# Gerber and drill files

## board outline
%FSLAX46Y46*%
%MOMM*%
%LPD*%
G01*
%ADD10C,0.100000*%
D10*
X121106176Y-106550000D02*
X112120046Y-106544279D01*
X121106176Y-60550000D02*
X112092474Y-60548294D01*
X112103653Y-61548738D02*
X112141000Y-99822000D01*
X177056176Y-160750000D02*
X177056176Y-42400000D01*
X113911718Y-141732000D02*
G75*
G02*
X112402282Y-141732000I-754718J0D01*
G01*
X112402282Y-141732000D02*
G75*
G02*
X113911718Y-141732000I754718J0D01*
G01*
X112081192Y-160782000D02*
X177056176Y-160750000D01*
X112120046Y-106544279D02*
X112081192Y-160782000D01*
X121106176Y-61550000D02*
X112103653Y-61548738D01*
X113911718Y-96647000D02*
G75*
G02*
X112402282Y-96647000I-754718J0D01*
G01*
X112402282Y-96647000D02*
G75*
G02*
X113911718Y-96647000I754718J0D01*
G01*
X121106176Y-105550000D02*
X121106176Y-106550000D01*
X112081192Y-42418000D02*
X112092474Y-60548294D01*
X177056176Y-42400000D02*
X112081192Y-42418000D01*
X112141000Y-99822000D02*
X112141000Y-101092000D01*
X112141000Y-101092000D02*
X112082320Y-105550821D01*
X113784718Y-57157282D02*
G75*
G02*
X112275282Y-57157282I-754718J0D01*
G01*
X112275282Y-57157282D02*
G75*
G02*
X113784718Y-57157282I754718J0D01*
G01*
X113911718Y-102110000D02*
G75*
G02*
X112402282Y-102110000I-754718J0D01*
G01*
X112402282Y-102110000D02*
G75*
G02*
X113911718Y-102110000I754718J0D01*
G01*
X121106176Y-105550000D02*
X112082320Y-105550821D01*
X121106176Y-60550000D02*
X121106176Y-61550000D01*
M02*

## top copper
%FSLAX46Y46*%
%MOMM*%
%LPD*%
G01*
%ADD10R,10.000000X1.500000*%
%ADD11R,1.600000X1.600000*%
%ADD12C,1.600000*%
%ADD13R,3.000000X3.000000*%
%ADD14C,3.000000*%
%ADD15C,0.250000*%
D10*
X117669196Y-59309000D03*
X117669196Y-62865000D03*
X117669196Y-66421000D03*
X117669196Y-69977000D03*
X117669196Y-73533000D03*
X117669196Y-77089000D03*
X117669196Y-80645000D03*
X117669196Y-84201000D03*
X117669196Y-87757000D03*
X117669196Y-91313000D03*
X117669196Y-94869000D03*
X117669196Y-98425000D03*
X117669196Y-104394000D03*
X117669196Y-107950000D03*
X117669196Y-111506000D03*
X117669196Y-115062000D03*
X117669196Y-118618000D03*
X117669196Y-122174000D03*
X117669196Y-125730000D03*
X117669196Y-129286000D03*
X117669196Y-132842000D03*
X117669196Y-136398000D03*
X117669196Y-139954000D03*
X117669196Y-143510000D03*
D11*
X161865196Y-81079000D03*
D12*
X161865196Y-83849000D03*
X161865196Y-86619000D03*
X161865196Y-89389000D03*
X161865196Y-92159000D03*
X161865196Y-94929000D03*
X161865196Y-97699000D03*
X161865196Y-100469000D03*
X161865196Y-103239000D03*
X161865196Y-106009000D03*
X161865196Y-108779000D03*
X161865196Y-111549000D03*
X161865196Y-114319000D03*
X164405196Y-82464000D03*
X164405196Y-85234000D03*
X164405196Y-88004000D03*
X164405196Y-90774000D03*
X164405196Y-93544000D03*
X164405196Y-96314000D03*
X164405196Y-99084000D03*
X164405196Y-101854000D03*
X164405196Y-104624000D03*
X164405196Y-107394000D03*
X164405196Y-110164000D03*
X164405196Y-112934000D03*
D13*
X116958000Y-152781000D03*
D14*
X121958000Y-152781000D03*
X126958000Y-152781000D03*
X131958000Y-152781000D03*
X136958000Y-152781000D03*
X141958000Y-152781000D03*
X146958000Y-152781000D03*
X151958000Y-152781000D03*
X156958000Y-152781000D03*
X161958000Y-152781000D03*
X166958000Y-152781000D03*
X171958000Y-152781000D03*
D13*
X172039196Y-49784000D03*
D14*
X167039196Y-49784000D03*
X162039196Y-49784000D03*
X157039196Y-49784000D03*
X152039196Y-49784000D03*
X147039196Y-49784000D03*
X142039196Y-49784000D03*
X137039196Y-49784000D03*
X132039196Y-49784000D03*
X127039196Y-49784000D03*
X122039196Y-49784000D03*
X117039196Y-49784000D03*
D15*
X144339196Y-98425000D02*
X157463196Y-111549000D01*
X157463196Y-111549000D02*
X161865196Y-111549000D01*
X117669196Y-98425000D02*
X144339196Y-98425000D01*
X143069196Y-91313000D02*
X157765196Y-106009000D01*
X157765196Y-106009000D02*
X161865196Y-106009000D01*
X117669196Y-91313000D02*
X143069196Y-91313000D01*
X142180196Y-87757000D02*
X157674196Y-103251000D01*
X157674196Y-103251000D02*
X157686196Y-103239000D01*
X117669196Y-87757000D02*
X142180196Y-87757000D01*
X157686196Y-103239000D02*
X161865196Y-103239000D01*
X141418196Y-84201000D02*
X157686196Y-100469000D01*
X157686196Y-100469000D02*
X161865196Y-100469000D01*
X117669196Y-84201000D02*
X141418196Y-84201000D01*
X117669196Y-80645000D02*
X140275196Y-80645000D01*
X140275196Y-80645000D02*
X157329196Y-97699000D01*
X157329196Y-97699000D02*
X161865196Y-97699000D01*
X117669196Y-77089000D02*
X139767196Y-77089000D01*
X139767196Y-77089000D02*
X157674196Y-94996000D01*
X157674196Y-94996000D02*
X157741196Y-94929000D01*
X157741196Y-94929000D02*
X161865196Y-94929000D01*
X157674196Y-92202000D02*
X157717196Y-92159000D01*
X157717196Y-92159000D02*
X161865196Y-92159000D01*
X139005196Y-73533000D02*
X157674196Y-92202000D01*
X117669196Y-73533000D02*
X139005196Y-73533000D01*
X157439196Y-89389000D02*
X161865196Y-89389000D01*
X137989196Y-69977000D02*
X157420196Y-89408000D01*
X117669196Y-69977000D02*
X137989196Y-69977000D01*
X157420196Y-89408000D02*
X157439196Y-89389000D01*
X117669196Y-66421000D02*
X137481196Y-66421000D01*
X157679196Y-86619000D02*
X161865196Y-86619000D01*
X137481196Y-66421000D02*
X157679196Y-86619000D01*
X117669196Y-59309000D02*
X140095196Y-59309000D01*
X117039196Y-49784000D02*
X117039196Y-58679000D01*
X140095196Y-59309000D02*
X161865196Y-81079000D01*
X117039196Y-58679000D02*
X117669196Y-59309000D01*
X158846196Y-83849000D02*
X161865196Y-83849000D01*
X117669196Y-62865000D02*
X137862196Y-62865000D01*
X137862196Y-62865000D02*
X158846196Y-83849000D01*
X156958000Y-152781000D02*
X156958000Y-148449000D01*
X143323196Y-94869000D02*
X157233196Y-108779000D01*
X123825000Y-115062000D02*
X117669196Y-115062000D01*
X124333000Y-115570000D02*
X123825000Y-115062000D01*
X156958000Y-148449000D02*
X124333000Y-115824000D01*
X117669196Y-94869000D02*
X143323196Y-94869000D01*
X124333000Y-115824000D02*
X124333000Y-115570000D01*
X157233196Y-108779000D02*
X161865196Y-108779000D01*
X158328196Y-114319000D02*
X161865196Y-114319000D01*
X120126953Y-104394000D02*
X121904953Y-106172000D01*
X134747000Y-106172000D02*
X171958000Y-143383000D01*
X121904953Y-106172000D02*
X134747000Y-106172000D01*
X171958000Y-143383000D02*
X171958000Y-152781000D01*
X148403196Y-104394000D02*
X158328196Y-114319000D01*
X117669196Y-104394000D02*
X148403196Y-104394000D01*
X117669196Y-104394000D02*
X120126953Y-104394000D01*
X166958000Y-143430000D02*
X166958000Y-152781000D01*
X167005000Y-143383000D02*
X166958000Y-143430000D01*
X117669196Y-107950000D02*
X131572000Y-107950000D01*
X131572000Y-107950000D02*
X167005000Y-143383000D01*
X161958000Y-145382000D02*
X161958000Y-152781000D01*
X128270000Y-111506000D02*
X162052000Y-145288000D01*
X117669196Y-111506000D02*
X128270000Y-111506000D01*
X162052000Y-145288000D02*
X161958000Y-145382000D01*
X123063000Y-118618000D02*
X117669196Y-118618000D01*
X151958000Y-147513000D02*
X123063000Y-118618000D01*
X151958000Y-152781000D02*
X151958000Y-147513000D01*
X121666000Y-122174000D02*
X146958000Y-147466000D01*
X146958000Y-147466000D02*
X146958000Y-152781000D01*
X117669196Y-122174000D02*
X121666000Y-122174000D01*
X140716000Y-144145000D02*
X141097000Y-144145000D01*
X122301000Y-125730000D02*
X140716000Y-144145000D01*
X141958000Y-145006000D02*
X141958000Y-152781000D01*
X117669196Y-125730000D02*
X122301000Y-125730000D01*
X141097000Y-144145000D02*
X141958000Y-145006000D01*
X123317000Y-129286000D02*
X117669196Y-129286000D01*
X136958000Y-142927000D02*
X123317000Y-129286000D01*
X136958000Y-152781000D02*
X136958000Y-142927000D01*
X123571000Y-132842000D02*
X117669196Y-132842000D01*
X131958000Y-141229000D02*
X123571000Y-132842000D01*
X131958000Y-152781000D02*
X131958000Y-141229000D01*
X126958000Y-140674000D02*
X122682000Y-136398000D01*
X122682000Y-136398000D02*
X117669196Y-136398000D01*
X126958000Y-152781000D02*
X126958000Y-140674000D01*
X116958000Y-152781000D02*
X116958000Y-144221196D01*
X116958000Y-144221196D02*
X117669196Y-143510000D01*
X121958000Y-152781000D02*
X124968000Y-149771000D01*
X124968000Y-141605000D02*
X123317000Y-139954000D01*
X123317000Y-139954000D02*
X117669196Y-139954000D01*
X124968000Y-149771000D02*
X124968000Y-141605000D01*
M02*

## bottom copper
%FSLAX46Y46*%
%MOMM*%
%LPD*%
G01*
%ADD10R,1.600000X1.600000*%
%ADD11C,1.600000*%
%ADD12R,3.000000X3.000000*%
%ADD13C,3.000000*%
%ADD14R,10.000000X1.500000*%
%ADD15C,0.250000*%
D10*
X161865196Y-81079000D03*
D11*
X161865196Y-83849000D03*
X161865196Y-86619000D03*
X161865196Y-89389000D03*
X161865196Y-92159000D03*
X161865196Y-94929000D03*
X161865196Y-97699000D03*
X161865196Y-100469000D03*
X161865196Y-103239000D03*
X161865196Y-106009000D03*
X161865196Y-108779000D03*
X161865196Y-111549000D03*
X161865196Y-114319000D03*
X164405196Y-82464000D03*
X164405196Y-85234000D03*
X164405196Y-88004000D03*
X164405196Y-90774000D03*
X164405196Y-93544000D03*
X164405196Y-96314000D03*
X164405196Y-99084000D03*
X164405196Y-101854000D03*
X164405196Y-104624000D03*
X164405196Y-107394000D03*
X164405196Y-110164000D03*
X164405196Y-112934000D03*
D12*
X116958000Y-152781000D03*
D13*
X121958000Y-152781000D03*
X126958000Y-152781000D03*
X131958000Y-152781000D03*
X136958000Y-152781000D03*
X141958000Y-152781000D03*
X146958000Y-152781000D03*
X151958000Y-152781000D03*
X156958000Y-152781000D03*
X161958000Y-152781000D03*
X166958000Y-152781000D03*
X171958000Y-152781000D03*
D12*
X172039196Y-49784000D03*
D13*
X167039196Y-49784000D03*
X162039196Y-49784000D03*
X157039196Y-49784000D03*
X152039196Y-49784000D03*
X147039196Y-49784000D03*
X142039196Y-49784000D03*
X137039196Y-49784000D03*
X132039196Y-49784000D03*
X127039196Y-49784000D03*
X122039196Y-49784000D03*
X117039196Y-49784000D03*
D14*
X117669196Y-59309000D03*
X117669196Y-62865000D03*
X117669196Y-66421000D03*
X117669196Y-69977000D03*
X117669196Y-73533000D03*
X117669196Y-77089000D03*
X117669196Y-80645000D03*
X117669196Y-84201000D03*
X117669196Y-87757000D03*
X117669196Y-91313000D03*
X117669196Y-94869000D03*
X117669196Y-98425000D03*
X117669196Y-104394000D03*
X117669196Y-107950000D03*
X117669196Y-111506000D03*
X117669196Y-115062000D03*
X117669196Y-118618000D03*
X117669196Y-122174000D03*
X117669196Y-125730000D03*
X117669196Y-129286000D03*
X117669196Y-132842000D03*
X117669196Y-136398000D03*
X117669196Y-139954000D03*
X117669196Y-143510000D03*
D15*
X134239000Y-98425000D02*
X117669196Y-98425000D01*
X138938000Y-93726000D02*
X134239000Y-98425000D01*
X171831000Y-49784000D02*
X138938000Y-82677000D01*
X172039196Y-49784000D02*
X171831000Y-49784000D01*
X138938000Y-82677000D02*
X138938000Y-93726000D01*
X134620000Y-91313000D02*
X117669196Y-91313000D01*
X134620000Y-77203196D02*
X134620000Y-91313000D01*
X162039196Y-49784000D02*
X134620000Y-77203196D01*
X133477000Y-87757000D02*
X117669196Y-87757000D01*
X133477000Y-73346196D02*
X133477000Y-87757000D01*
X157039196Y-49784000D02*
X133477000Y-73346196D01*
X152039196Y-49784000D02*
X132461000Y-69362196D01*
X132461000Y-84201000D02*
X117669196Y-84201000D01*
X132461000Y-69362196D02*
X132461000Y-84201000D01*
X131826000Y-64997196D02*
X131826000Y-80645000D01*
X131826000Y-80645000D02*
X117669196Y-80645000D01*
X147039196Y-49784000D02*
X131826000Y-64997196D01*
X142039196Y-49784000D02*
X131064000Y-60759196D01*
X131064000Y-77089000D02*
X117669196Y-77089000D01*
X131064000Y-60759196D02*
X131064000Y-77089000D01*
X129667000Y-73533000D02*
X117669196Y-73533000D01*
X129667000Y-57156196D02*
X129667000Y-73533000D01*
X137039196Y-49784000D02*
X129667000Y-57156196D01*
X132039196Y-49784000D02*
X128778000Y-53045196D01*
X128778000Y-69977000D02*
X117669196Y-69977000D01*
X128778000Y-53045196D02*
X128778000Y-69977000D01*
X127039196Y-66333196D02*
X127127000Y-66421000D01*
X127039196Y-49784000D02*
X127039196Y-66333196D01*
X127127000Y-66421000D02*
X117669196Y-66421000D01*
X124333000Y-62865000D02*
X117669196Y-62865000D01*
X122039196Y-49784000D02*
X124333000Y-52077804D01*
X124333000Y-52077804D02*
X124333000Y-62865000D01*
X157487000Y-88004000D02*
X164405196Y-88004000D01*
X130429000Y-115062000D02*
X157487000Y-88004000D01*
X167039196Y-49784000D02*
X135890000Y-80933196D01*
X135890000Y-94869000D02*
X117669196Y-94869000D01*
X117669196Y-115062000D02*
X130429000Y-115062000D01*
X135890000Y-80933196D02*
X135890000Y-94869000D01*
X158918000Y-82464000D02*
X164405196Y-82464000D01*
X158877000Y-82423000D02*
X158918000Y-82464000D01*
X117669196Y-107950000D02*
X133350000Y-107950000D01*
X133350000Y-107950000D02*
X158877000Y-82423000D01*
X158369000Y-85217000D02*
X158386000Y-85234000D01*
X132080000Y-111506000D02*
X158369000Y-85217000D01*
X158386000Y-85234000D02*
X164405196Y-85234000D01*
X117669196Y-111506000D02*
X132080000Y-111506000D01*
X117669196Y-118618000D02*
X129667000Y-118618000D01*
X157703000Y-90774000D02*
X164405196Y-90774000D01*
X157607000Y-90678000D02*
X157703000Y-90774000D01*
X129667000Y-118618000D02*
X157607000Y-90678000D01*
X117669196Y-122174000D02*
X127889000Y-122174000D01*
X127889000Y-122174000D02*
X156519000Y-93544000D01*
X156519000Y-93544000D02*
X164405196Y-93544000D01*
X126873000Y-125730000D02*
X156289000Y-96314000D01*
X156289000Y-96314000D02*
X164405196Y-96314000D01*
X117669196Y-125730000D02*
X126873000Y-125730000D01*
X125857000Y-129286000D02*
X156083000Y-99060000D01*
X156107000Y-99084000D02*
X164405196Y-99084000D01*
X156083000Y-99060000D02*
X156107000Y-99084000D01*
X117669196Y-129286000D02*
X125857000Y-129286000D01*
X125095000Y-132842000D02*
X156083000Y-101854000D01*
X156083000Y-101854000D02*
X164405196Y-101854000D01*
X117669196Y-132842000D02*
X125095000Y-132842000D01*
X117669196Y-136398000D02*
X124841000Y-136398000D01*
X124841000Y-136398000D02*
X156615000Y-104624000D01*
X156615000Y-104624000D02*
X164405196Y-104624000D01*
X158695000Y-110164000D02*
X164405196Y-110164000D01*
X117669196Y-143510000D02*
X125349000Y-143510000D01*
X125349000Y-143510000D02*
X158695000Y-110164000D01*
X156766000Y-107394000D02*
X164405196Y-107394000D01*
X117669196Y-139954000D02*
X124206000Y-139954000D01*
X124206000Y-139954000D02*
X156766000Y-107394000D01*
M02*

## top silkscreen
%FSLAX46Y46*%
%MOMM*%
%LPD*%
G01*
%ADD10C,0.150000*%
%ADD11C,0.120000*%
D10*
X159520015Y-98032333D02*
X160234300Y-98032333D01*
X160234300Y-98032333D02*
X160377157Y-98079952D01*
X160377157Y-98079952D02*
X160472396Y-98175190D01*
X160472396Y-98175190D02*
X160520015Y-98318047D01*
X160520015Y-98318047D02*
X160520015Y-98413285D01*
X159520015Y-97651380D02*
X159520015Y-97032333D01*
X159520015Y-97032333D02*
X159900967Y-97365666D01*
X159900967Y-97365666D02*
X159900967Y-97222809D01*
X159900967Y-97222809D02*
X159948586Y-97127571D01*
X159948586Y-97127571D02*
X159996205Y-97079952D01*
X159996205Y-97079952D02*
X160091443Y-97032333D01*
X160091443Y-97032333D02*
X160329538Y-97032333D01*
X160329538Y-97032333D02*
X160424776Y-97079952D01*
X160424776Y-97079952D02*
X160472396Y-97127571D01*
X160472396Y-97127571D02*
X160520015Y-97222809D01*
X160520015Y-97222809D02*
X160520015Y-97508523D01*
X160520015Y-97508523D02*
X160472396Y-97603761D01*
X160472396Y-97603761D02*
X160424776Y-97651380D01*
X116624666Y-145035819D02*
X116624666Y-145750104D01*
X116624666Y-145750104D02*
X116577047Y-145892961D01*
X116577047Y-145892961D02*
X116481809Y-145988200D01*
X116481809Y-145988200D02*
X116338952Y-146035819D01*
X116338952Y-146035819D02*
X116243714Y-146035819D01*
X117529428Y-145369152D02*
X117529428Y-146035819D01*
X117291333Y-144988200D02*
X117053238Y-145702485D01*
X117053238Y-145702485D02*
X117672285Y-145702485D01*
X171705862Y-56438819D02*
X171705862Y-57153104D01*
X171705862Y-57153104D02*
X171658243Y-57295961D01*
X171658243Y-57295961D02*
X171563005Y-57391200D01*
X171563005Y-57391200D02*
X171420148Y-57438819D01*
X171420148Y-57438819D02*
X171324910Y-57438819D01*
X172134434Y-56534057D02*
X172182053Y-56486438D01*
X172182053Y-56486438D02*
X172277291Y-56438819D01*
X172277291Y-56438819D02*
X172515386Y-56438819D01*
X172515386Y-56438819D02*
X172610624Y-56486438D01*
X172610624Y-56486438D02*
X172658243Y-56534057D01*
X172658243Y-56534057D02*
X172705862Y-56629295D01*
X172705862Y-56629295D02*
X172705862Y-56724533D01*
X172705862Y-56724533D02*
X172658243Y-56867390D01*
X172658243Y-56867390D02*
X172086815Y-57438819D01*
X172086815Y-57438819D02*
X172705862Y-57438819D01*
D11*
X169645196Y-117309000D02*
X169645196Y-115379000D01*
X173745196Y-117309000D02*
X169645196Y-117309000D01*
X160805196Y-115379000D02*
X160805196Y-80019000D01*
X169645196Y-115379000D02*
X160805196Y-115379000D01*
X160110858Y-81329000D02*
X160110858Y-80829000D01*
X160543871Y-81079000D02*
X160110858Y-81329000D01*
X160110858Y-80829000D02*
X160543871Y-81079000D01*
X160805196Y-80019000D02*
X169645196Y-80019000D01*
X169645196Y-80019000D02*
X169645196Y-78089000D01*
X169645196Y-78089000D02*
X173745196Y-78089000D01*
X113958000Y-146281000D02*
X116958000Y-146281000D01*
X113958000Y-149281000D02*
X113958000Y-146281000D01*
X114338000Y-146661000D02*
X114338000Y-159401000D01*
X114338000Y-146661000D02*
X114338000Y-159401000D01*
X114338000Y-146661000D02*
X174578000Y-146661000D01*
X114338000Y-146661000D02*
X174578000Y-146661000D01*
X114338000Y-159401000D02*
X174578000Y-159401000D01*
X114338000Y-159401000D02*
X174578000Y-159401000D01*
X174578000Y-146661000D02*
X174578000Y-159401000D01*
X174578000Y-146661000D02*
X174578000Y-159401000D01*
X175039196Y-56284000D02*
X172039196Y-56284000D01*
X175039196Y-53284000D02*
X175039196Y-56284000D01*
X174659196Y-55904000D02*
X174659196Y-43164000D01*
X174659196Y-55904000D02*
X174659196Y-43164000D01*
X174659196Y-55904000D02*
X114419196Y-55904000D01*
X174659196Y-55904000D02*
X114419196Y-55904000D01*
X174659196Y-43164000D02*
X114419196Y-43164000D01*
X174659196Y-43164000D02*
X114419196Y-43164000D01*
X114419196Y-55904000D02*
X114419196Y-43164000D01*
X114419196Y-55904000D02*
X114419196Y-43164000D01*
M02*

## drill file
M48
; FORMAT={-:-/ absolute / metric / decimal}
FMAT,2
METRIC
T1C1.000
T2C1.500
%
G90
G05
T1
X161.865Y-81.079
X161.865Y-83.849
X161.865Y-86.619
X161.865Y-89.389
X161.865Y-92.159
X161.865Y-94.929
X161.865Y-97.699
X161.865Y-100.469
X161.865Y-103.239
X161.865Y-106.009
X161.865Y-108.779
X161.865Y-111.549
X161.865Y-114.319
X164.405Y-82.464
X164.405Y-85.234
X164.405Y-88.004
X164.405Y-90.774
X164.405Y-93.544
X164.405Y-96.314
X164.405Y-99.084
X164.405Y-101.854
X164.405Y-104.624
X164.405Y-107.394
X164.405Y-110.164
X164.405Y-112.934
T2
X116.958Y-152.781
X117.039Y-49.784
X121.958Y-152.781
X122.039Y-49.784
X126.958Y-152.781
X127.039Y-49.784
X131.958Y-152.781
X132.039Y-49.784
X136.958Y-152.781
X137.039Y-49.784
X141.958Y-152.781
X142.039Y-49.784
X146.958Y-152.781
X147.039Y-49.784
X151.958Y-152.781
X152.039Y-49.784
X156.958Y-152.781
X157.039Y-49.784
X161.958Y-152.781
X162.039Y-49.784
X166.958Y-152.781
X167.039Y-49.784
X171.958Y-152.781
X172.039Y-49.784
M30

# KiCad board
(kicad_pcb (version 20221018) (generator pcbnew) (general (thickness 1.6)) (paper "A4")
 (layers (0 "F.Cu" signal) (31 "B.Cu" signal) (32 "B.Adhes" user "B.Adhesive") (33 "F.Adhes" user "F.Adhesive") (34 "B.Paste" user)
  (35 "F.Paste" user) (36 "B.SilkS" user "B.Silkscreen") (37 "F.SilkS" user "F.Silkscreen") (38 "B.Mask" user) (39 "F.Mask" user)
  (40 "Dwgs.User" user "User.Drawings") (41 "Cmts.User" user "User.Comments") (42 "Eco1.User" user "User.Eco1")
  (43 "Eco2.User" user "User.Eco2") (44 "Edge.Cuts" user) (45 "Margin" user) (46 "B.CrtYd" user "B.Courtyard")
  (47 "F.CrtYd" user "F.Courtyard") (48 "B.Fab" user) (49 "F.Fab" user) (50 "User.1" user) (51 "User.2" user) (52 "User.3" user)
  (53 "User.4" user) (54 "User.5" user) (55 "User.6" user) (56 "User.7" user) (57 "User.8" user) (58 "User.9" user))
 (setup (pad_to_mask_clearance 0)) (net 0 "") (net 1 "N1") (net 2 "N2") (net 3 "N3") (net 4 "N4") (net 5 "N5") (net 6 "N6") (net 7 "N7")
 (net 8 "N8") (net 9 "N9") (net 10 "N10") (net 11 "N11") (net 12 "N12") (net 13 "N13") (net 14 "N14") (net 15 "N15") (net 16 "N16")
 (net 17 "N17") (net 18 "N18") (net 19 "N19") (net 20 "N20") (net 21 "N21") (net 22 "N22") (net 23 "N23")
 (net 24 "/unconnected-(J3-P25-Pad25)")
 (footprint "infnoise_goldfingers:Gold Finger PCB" (layer "F.Cu") (at 123.257196 78.867 -90)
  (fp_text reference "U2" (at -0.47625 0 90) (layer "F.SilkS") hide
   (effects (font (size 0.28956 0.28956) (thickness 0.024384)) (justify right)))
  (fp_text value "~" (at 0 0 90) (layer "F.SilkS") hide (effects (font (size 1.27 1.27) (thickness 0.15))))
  (pad "1" smd rect (at -19.558 5.588 270) (size 1.5 10) (layers "F.Cu" "F.Paste" "F.Mask") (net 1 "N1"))
  (pad "2" smd rect (at -16.002 5.588 270) (size 1.5 10) (layers "F.Cu" "F.Paste" "F.Mask") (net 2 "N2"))
  (pad "3" smd rect (at -12.446 5.588 270) (size 1.5 10) (layers "F.Cu" "F.Paste" "F.Mask") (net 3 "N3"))
  (pad "4" smd rect (at -8.89 5.588 270) (size 1.5 10) (layers "F.Cu" "F.Paste" "F.Mask") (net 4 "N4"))
  (pad "5" smd rect (at -5.334 5.588 270) (size 1.5 10) (layers "F.Cu" "F.Paste" "F.Mask") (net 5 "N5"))
  (pad "6" smd rect (at -1.778 5.588 270) (size 1.5 10) (layers "F.Cu" "F.Paste" "F.Mask") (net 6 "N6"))
  (pad "7" smd rect (at 1.778 5.588 270) (size 1.5 10) (layers "F.Cu" "F.Paste" "F.Mask") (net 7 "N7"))
  (pad "8" smd rect (at 5.334 5.588 270) (size 1.5 10) (layers "F.Cu" "F.Paste" "F.Mask") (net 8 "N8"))
  (pad "9" smd rect (at 8.89 5.588 270) (size 1.5 10) (layers "F.Cu" "F.Paste" "F.Mask") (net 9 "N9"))
  (pad "10" smd rect (at 12.446 5.588 270) (size 1.5 10) (layers "F.Cu" "F.Paste" "F.Mask") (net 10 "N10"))
  (pad "11" smd rect (at 16.002 5.588 270) (size 1.5 10) (layers "F.Cu" "F.Paste" "F.Mask") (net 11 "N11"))
  (pad "12" smd rect (at 19.558 5.588 270) (size 1.5 10) (layers "F.Cu" "F.Paste" "F.Mask") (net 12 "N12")))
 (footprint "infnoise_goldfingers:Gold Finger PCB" (layer "F.Cu") (at 123.257196 123.952 -90)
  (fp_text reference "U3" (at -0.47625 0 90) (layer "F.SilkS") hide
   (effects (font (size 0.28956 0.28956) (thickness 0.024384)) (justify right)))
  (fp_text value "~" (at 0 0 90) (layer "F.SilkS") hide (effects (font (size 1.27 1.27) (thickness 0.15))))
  (pad "1" smd rect (at -19.558 5.588 270) (size 1.5 10) (layers "F.Cu" "F.Paste" "F.Mask") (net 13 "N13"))
  (pad "2" smd rect (at -16.002 5.588 270) (size 1.5 10) (layers "F.Cu" "F.Paste" "F.Mask") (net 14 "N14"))
  (pad "3" smd rect (at -12.446 5.588 270) (size 1.5 10) (layers "F.Cu" "F.Paste" "F.Mask") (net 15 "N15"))
  (pad "4" smd rect (at -8.89 5.588 270) (size 1.5 10) (layers "F.Cu" "F.Paste" "F.Mask") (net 11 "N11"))
  (pad "5" smd rect (at -5.334 5.588 270) (size 1.5 10) (layers "F.Cu" "F.Paste" "F.Mask") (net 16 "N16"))
  (pad "6" smd rect (at -1.778 5.588 270) (size 1.5 10) (layers "F.Cu" "F.Paste" "F.Mask") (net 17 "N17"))
  (pad "7" smd rect (at 1.778 5.588 270) (size 1.5 10) (layers "F.Cu" "F.Paste" "F.Mask") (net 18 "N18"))
  (pad "8" smd rect (at 5.334 5.588 270) (size 1.5 10) (layers "F.Cu" "F.Paste" "F.Mask") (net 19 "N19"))
  (pad "9" smd rect (at 8.89 5.588 270) (size 1.5 10) (layers "F.Cu" "F.Paste" "F.Mask") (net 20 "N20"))
  (pad "10" smd rect (at 12.446 5.588 270) (size 1.5 10) (layers "F.Cu" "F.Paste" "F.Mask") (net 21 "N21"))
  (pad "11" smd rect (at 16.002 5.588 270) (size 1.5 10) (layers "F.Cu" "F.Paste" "F.Mask") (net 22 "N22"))
  (pad "12" smd rect (at 19.558 5.588 270) (size 1.5 10) (layers "F.Cu" "F.Paste" "F.Mask") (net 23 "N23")))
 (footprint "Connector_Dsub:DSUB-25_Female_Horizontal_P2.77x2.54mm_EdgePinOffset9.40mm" (layer "F.Cu") (at 161.865196 81.079 90)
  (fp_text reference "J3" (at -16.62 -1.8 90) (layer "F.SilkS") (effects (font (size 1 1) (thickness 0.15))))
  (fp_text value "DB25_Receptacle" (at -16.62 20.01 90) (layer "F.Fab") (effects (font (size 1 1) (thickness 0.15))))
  (fp_line (start -36.23 7.78) (end -34.3 7.78) (stroke (width 0.12) (type solid)) (layer "F.SilkS"))
  (fp_line (start -36.23 11.88) (end -36.23 7.78) (stroke (width 0.12) (type solid)) (layer "F.SilkS"))
  (fp_line (start -34.3 -1.06) (end 1.06 -1.06) (stroke (width 0.12) (type solid)) (layer "F.SilkS"))
  (fp_line (start -34.3 7.78) (end -34.3 -1.06) (stroke (width 0.12) (type solid)) (layer "F.SilkS"))
  (fp_line (start -0.25 -1.754338) (end 0.25 -1.754338) (stroke (width 0.12) (type solid)) (layer "F.SilkS"))
  (fp_line (start 0 -1.321325) (end -0.25 -1.754338) (stroke (width 0.12) (type solid)) (layer "F.SilkS"))
  (fp_line (start 0.25 -1.754338) (end 0 -1.321325) (stroke (width 0.12) (type solid)) (layer "F.SilkS"))
  (fp_line (start 1.06 -1.06) (end 1.06 7.78) (stroke (width 0.12) (type solid)) (layer "F.SilkS"))
  (fp_line (start 1.06 7.78) (end 2.99 7.78) (stroke (width 0.12) (type solid)) (layer "F.SilkS"))
  (fp_line (start 2.99 7.78) (end 2.99 11.88) (stroke (width 0.12) (type solid)) (layer "F.SilkS"))
  (pad "1" thru_hole rect (at 0 0 90) (size 1.6 1.6) (drill 1) (layers "*.Cu" "*.Mask") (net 1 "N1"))
  (pad "2" thru_hole circle (at -2.77 0 90) (size 1.6 1.6) (drill 1) (layers "*.Cu" "*.Mask") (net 2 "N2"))
  (pad "3" thru_hole circle (at -5.54 0 90) (size 1.6 1.6) (drill 1) (layers "*.Cu" "*.Mask") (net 3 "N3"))
  (pad "4" thru_hole circle (at -8.31 0 90) (size 1.6 1.6) (drill 1) (layers "*.Cu" "*.Mask") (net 4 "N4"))
  (pad "5" thru_hole circle (at -11.08 0 90) (size 1.6 1.6) (drill 1) (layers "*.Cu" "*.Mask") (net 5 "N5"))
  (pad "6" thru_hole circle (at -13.85 0 90) (size 1.6 1.6) (drill 1) (layers "*.Cu" "*.Mask") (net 6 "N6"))
  (pad "7" thru_hole circle (at -16.62 0 90) (size 1.6 1.6) (drill 1) (layers "*.Cu" "*.Mask") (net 7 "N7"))
  (pad "8" thru_hole circle (at -19.39 0 90) (size 1.6 1.6) (drill 1) (layers "*.Cu" "*.Mask") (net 8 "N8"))
  (pad "9" thru_hole circle (at -22.16 0 90) (size 1.6 1.6) (drill 1) (layers "*.Cu" "*.Mask") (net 9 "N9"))
  (pad "10" thru_hole circle (at -24.93 0 90) (size 1.6 1.6) (drill 1) (layers "*.Cu" "*.Mask") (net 10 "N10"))
  (pad "11" thru_hole circle (at -27.7 0 90) (size 1.6 1.6) (drill 1) (layers "*.Cu" "*.Mask") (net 11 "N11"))
  (pad "12" thru_hole circle (at -30.47 0 90) (size 1.6 1.6) (drill 1) (layers "*.Cu" "*.Mask") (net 12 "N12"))
  (pad "13" thru_hole circle (at -33.24 0 90) (size 1.6 1.6) (drill 1) (layers "*.Cu" "*.Mask") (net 13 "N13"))
  (pad "14" thru_hole circle (at -1.385 2.54 90) (size 1.6 1.6) (drill 1) (layers "*.Cu" "*.Mask") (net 14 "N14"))
  (pad "15" thru_hole circle (at -4.155 2.54 90) (size 1.6 1.6) (drill 1) (layers "*.Cu" "*.Mask") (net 15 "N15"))
  (pad "16" thru_hole circle (at -6.925 2.54 90) (size 1.6 1.6) (drill 1) (layers "*.Cu" "*.Mask") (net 11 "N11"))
  (pad "17" thru_hole circle (at -9.695 2.54 90) (size 1.6 1.6) (drill 1) (layers "*.Cu" "*.Mask") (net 16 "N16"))
  (pad "18" thru_hole circle (at -12.465 2.54 90) (size 1.6 1.6) (drill 1) (layers "*.Cu" "*.Mask") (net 17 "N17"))
  (pad "19" thru_hole circle (at -15.235 2.54 90) (size 1.6 1.6) (drill 1) (layers "*.Cu" "*.Mask") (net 18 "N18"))
  (pad "20" thru_hole circle (at -18.005 2.54 90) (size 1.6 1.6) (drill 1) (layers "*.Cu" "*.Mask") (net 19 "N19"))
  (pad "21" thru_hole circle (at -20.775 2.54 90) (size 1.6 1.6) (drill 1) (layers "*.Cu" "*.Mask") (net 20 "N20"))
  (pad "22" thru_hole circle (at -23.545 2.54 90) (size 1.6 1.6) (drill 1) (layers "*.Cu" "*.Mask") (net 21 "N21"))
  (pad "23" thru_hole circle (at -26.315 2.54 90) (size 1.6 1.6) (drill 1) (layers "*.Cu" "*.Mask") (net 22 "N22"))
  (pad "24" thru_hole circle (at -29.085 2.54 90) (size 1.6 1.6) (drill 1) (layers "*.Cu" "*.Mask") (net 23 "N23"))
  (pad "25" thru_hole circle (at -31.855 2.54 90) (size 1.6 1.6) (drill 1) (layers "*.Cu" "*.Mask") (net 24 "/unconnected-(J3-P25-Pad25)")))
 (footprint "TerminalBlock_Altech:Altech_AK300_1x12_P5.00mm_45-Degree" (layer "F.Cu") (at 116.958 152.781)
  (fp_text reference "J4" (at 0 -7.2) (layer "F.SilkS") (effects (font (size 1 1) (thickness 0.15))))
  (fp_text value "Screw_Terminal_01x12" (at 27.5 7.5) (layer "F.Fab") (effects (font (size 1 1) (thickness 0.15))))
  (fp_line (start -3 -6.5) (end 0 -6.5) (stroke (width 0.12) (type solid)) (layer "F.SilkS"))
  (fp_line (start -3 -3.5) (end -3 -6.5) (stroke (width 0.12) (type solid)) (layer "F.SilkS"))
  (fp_line (start -2.62 -6.12) (end -2.62 6.62) (stroke (width 0.12) (type solid)) (layer "F.SilkS"))
  (fp_line (start -2.62 -6.12) (end -2.62 6.62) (stroke (width 0.12) (type solid)) (layer "F.SilkS"))
  (fp_line (start -2.62 -6.12) (end 57.62 -6.12) (stroke (width 0.12) (type solid)) (layer "F.SilkS"))
  (fp_line (start -2.62 -6.12) (end 57.62 -6.12) (stroke (width 0.12) (type solid)) (layer "F.SilkS"))
  (fp_line (start -2.62 6.62) (end 57.62 6.62) (stroke (width 0.12) (type solid)) (layer "F.SilkS"))
  (fp_line (start -2.62 6.62) (end 57.62 6.62) (stroke (width 0.12) (type solid)) (layer "F.SilkS"))
  (fp_line (start 57.62 -6.12) (end 57.62 6.62) (stroke (width 0.12) (type solid)) (layer "F.SilkS"))
  (fp_line (start 57.62 -6.12) (end 57.62 6.62) (stroke (width 0.12) (type solid)) (layer "F.SilkS"))
  (pad "1" thru_hole rect (at 0 0) (size 3 3) (drill 1.5) (layers "*.Cu" "*.Mask") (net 23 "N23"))
  (pad "2" thru_hole circle (at 5 0) (size 3 3) (drill 1.5) (layers "*.Cu" "*.Mask") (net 22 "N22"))
  (pad "3" thru_hole circle (at 10 0) (size 3 3) (drill 1.5) (layers "*.Cu" "*.Mask") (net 21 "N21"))
  (pad "4" thru_hole circle (at 15 0) (size 3 3) (drill 1.5) (layers "*.Cu" "*.Mask") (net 20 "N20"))
  (pad "5" thru_hole circle (at 20 0) (size 3 3) (drill 1.5) (layers "*.Cu" "*.Mask") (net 19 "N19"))
  (pad "6" thru_hole circle (at 25 0) (size 3 3) (drill 1.5) (layers "*.Cu" "*.Mask") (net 18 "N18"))
  (pad "7" thru_hole circle (at 30 0) (size 3 3) (drill 1.5) (layers "*.Cu" "*.Mask") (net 17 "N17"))
  (pad "8" thru_hole circle (at 35 0) (size 3 3) (drill 1.5) (layers "*.Cu" "*.Mask") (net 16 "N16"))
  (pad "9" thru_hole circle (at 40 0) (size 3 3) (drill 1.5) (layers "*.Cu" "*.Mask") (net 11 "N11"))
  (pad "10" thru_hole circle (at 45 0) (size 3 3) (drill 1.5) (layers "*.Cu" "*.Mask") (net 15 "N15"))
  (pad "11" thru_hole circle (at 50 0) (size 3 3) (drill 1.5) (layers "*.Cu" "*.Mask") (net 14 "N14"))
  (pad "12" thru_hole circle (at 55 0) (size 3 3) (drill 1.5) (layers "*.Cu" "*.Mask") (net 13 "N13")))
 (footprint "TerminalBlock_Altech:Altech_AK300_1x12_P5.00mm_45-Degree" (layer "F.Cu") (at 172.039196 49.784 180)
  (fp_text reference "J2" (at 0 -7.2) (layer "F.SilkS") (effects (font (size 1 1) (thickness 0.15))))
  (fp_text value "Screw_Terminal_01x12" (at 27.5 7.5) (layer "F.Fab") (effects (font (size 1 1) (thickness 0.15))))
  (fp_line (start -3 -6.5) (end 0 -6.5) (stroke (width 0.12) (type solid)) (layer "F.SilkS"))
  (fp_line (start -3 -3.5) (end -3 -6.5) (stroke (width 0.12) (type solid)) (layer "F.SilkS"))
  (fp_line (start -2.62 -6.12) (end -2.62 6.62) (stroke (width 0.12) (type solid)) (layer "F.SilkS"))
  (fp_line (start -2.62 -6.12) (end -2.62 6.62) (stroke (width 0.12) (type solid)) (layer "F.SilkS"))
  (fp_line (start -2.62 -6.12) (end 57.62 -6.12) (stroke (width 0.12) (type solid)) (layer "F.SilkS"))
  (fp_line (start -2.62 -6.12) (end 57.62 -6.12) (stroke (width 0.12) (type solid)) (layer "F.SilkS"))
  (fp_line (start -2.62 6.62) (end 57.62 6.62) (stroke (width 0.12) (type solid)) (layer "F.SilkS"))
  (fp_line (start -2.62 6.62) (end 57.62 6.62) (stroke (width 0.12) (type solid)) (layer "F.SilkS"))
  (fp_line (start 57.62 -6.12) (end 57.62 6.62) (stroke (width 0.12) (type solid)) (layer "F.SilkS"))
  (fp_line (start 57.62 -6.12) (end 57.62 6.62) (stroke (width 0.12) (type solid)) (layer "F.SilkS"))
  (pad "1" thru_hole rect (at 0 0 180) (size 3 3) (drill 1.5) (layers "*.Cu" "*.Mask") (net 12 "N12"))
  (pad "2" thru_hole circle (at 5 0 180) (size 3 3) (drill 1.5) (layers "*.Cu" "*.Mask") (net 11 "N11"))
  (pad "3" thru_hole circle (at 10 0 180) (size 3 3) (drill 1.5) (layers "*.Cu" "*.Mask") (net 10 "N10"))
  (pad "4" thru_hole circle (at 15 0 180) (size 3 3) (drill 1.5) (layers "*.Cu" "*.Mask") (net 9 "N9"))
  (pad "5" thru_hole circle (at 20 0 180) (size 3 3) (drill 1.5) (layers "*.Cu" "*.Mask") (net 8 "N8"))
  (pad "6" thru_hole circle (at 25 0 180) (size 3 3) (drill 1.5) (layers "*.Cu" "*.Mask") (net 7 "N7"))
  (pad "7" thru_hole circle (at 30 0 180) (size 3 3) (drill 1.5) (layers "*.Cu" "*.Mask") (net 6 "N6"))
  (pad "8" thru_hole circle (at 35 0 180) (size 3 3) (drill 1.5) (layers "*.Cu" "*.Mask") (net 5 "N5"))
  (pad "9" thru_hole circle (at 40 0 180) (size 3 3) (drill 1.5) (layers "*.Cu" "*.Mask") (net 4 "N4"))
  (pad "10" thru_hole circle (at 45 0 180) (size 3 3) (drill 1.5) (layers "*.Cu" "*.Mask") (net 3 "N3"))
  (pad "11" thru_hole circle (at 50 0 180) (size 3 3) (drill 1.5) (layers "*.Cu" "*.Mask") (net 2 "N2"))
  (pad "12" thru_hole circle (at 55 0 180) (size 3 3) (drill 1.5) (layers "*.Cu" "*.Mask") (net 1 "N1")))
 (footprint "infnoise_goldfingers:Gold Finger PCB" (layer "B.Cu") (at 112.081196 78.867 -90)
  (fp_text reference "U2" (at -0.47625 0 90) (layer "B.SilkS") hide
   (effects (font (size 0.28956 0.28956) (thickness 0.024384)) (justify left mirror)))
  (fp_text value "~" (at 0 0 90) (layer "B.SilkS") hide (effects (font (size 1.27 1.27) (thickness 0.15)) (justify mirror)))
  (pad "1" smd rect (at -19.558 -5.588 270) (size 1.5 10) (layers "B.Cu" "B.Paste" "B.Mask") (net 1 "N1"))
  (pad "2" smd rect (at -16.002 -5.588 270) (size 1.5 10) (layers "B.Cu" "B.Paste" "B.Mask") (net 2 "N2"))
  (pad "3" smd rect (at -12.446 -5.588 270) (size 1.5 10) (layers "B.Cu" "B.Paste" "B.Mask") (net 3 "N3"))
  (pad "4" smd rect (at -8.89 -5.588 270) (size 1.5 10) (layers "B.Cu" "B.Paste" "B.Mask") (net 4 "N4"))
  (pad "5" smd rect (at -5.334 -5.588 270) (size 1.5 10) (layers "B.Cu" "B.Paste" "B.Mask") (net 5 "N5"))
  (pad "6" smd rect (at -1.778 -5.588 270) (size 1.5 10) (layers "B.Cu" "B.Paste" "B.Mask") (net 6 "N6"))
  (pad "7" smd rect (at 1.778 -5.588 270) (size 1.5 10) (layers "B.Cu" "B.Paste" "B.Mask") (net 7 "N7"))
  (pad "8" smd rect (at 5.334 -5.588 270) (size 1.5 10) (layers "B.Cu" "B.Paste" "B.Mask") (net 8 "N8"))
  (pad "9" smd rect (at 8.89 -5.588 270) (size 1.5 10) (layers "B.Cu" "B.Paste" "B.Mask") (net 9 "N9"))
  (pad "10" smd rect (at 12.446 -5.588 270) (size 1.5 10) (layers "B.Cu" "B.Paste" "B.Mask") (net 10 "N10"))
  (pad "11" smd rect (at 16.002 -5.588 270) (size 1.5 10) (layers "B.Cu" "B.Paste" "B.Mask") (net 11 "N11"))
  (pad "12" smd rect (at 19.558 -5.588 270) (size 1.5 10) (layers "B.Cu" "B.Paste" "B.Mask") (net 12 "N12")))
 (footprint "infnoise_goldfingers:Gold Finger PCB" (layer "B.Cu") (at 112.081196 123.952 -90)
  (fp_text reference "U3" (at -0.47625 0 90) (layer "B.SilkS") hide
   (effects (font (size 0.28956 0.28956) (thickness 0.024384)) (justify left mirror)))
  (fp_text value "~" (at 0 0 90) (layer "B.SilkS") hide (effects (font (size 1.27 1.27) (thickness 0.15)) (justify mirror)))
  (pad "1" smd rect (at -19.558 -5.588 270) (size 1.5 10) (layers "B.Cu" "B.Paste" "B.Mask") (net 13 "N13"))
  (pad "2" smd rect (at -16.002 -5.588 270) (size 1.5 10) (layers "B.Cu" "B.Paste" "B.Mask") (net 14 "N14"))
  (pad "3" smd rect (at -12.446 -5.588 270) (size 1.5 10) (layers "B.Cu" "B.Paste" "B.Mask") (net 15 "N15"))
  (pad "4" smd rect (at -8.89 -5.588 270) (size 1.5 10) (layers "B.Cu" "B.Paste" "B.Mask") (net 11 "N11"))
  (pad "5" smd rect (at -5.334 -5.588 270) (size 1.5 10) (layers "B.Cu" "B.Paste" "B.Mask") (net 16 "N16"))
  (pad "6" smd rect (at -1.778 -5.588 270) (size 1.5 10) (layers "B.Cu" "B.Paste" "B.Mask") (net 17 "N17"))
  (pad "7" smd rect (at 1.778 -5.588 270) (size 1.5 10) (layers "B.Cu" "B.Paste" "B.Mask") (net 18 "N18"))
  (pad "8" smd rect (at 5.334 -5.588 270) (size 1.5 10) (layers "B.Cu" "B.Paste" "B.Mask") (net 19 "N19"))
  (pad "9" smd rect (at 8.89 -5.588 270) (size 1.5 10) (layers "B.Cu" "B.Paste" "B.Mask") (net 20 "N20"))
  (pad "10" smd rect (at 12.446 -5.588 270) (size 1.5 10) (layers "B.Cu" "B.Paste" "B.Mask") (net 21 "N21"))
  (pad "11" smd rect (at 16.002 -5.588 270) (size 1.5 10) (layers "B.Cu" "B.Paste" "B.Mask") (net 22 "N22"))
  (pad "12" smd rect (at 19.558 -5.588 270) (size 1.5 10) (layers "B.Cu" "B.Paste" "B.Mask") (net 23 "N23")))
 (gr_line (start 121.106176 106.55) (end 112.120046 106.544279) (stroke (width 0.1) (type default)) (layer "Edge.Cuts"))
 (gr_line (start 121.106176 60.55) (end 112.092474 60.548294) (stroke (width 0.1) (type default)) (layer "Edge.Cuts"))
 (gr_line (start 112.103653 61.548738) (end 112.141 99.822) (stroke (width 0.1) (type default)) (layer "Edge.Cuts"))
 (gr_line (start 177.056176 160.75) (end 177.056176 42.4) (stroke (width 0.1) (type default)) (layer "Edge.Cuts"))
 (gr_circle (center 113.157 141.732) (end 113.557 142.372) (stroke (width 0.1) (type default)) (fill none) (layer "Edge.Cuts"))
 (gr_line (start 112.081192 160.782) (end 177.056176 160.75) (stroke (width 0.1) (type default)) (layer "Edge.Cuts"))
 (gr_line (start 112.120046 106.544279) (end 112.081192 160.782) (stroke (width 0.1) (type default)) (layer "Edge.Cuts"))
 (gr_line (start 121.106176 61.55) (end 112.103653 61.548738) (stroke (width 0.1) (type default)) (layer "Edge.Cuts"))
 (gr_circle (center 113.157 96.647) (end 113.557 97.287) (stroke (width 0.1) (type default)) (fill none) (layer "Edge.Cuts"))
 (gr_line (start 121.106176 105.55) (end 121.106176 106.55) (stroke (width 0.1) (type default)) (layer "Edge.Cuts"))
 (gr_line (start 112.081192 42.418) (end 112.092474 60.548294) (stroke (width 0.1) (type default)) (layer "Edge.Cuts"))
 (gr_line (start 177.056176 42.4) (end 112.081192 42.418) (stroke (width 0.1) (type default)) (layer "Edge.Cuts"))
 (gr_line (start 112.141 99.822) (end 112.141 101.092) (stroke (width 0.1) (type default)) (layer "Edge.Cuts"))
 (gr_line (start 112.141 101.092) (end 112.08232 105.550821) (stroke (width 0.1) (type default)) (layer "Edge.Cuts"))
 (gr_circle (center 113.03 57.157282) (end 113.43 57.797282) (stroke (width 0.1) (type default)) (fill none) (layer "Edge.Cuts"))
 (gr_circle (center 113.157 102.11) (end 113.557 102.75) (stroke (width 0.1) (type default)) (fill none) (layer "Edge.Cuts"))
 (gr_line (start 121.106176 105.55) (end 112.08232 105.550821) (stroke (width 0.1) (type default)) (layer "Edge.Cuts"))
 (gr_line (start 121.106176 60.55) (end 121.106176 61.55) (stroke (width 0.1) (type default)) (layer "Edge.Cuts"))
 (segment (start 144.339196 98.425) (end 157.463196 111.549) (width 0.25) (layer "F.Cu") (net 12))
 (segment (start 157.463196 111.549) (end 161.865196 111.549) (width 0.25) (layer "F.Cu") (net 12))
 (segment (start 117.669196 98.425) (end 144.339196 98.425) (width 0.25) (layer "F.Cu") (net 12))
 (segment (start 134.239 98.425) (end 117.669196 98.425) (width 0.25) (layer "B.Cu") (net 12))
 (segment (start 138.938 93.726) (end 134.239 98.425) (width 0.25) (layer "B.Cu") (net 12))
 (segment (start 171.831 49.784) (end 138.938 82.677) (width 0.25) (layer "B.Cu") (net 12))
 (segment (start 172.039196 49.784) (end 171.831 49.784) (width 0.25) (layer "B.Cu") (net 12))
 (segment (start 138.938 82.677) (end 138.938 93.726) (width 0.25) (layer "B.Cu") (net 12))
 (segment (start 143.069196 91.313) (end 157.765196 106.009) (width 0.25) (layer "F.Cu") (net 10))
 (segment (start 157.765196 106.009) (end 161.865196 106.009) (width 0.25) (layer "F.Cu") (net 10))
 (segment (start 117.669196 91.313) (end 143.069196 91.313) (width 0.25) (layer "F.Cu") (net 10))
 (segment (start 134.62 91.313) (end 117.669196 91.313) (width 0.25) (layer "B.Cu") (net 10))
 (segment (start 134.62 77.203196) (end 134.62 91.313) (width 0.25) (layer "B.Cu") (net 10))
 (segment (start 162.039196 49.784) (end 134.62 77.203196) (width 0.25) (layer "B.Cu") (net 10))
 (segment (start 142.180196 87.757) (end 157.674196 103.251) (width 0.25) (layer "F.Cu") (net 9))
 (segment (start 157.674196 103.251) (end 157.686196 103.239) (width 0.25) (layer "F.Cu") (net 9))
 (segment (start 117.669196 87.757) (end 142.180196 87.757) (width 0.25) (layer "F.Cu") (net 9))
 (segment (start 157.686196 103.239) (end 161.865196 103.239) (width 0.25) (layer "F.Cu") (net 9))
 (segment (start 133.477 87.757) (end 117.669196 87.757) (width 0.25) (layer "B.Cu") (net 9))
 (segment (start 133.477 73.346196) (end 133.477 87.757) (width 0.25) (layer "B.Cu") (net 9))
 (segment (start 157.039196 49.784) (end 133.477 73.346196) (width 0.25) (layer "B.Cu") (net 9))
 (segment (start 141.418196 84.201) (end 157.686196 100.469) (width 0.25) (layer "F.Cu") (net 8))
 (segment (start 157.686196 100.469) (end 161.865196 100.469) (width 0.25) (layer "F.Cu") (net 8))
 (segment (start 117.669196 84.201) (end 141.418196 84.201) (width 0.25) (layer "F.Cu") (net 8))
 (segment (start 152.039196 49.784) (end 132.461 69.362196) (width 0.25) (layer "B.Cu") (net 8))
 (segment (start 132.461 84.201) (end 117.669196 84.201) (width 0.25) (layer "B.Cu") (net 8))
 (segment (start 132.461 69.362196) (end 132.461 84.201) (width 0.25) (layer "B.Cu") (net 8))
 (segment (start 117.669196 80.645) (end 140.275196 80.645) (width 0.25) (layer "F.Cu") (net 7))
 (segment (start 140.275196 80.645) (end 157.329196 97.699) (width 0.25) (layer "F.Cu") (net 7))
 (segment (start 157.329196 97.699) (end 161.865196 97.699) (width 0.25) (layer "F.Cu") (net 7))
 (segment (start 131.826 64.997196) (end 131.826 80.645) (width 0.25) (layer "B.Cu") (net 7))
 (segment (start 131.826 80.645) (end 117.669196 80.645) (width 0.25) (layer "B.Cu") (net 7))
 (segment (start 147.039196 49.784) (end 131.826 64.997196) (width 0.25) (layer "B.Cu") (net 7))
 (segment (start 117.669196 77.089) (end 139.767196 77.089) (width 0.25) (layer "F.Cu") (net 6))
 (segment (start 139.767196 77.089) (end 157.674196 94.996) (width 0.25) (layer "F.Cu") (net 6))
 (segment (start 157.674196 94.996) (end 157.741196 94.929) (width 0.25) (layer "F.Cu") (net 6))
 (segment (start 157.741196 94.929) (end 161.865196 94.929) (width 0.25) (layer "F.Cu") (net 6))
 (segment (start 142.039196 49.784) (end 131.064 60.759196) (width 0.25) (layer "B.Cu") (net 6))
 (segment (start 131.064 77.089) (end 117.669196 77.089) (width 0.25) (layer "B.Cu") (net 6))
 (segment (start 131.064 60.759196) (end 131.064 77.089) (width 0.25) (layer "B.Cu") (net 6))
 (segment (start 157.674196 92.202) (end 157.717196 92.159) (width 0.25) (layer "F.Cu") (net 5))
 (segment (start 157.717196 92.159) (end 161.865196 92.159) (width 0.25) (layer "F.Cu") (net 5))
 (segment (start 139.005196 73.533) (end 157.674196 92.202) (width 0.25) (layer "F.Cu") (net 5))
 (segment (start 117.669196 73.533) (end 139.005196 73.533) (width 0.25) (layer "F.Cu") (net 5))
 (segment (start 129.667 73.533) (end 117.669196 73.533) (width 0.25) (layer "B.Cu") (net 5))
 (segment (start 129.667 57.156196) (end 129.667 73.533) (width 0.25) (layer "B.Cu") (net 5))
 (segment (start 137.039196 49.784) (end 129.667 57.156196) (width 0.25) (layer "B.Cu") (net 5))
 (segment (start 157.439196 89.389) (end 161.865196 89.389) (width 0.25) (layer "F.Cu") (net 4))
 (segment (start 137.989196 69.977) (end 157.420196 89.408) (width 0.25) (layer "F.Cu") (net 4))
 (segment (start 117.669196 69.977) (end 137.989196 69.977) (width 0.25) (layer "F.Cu") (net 4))
 (segment (start 157.420196 89.408) (end 157.439196 89.389) (width 0.25) (layer "F.Cu") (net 4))
 (segment (start 132.039196 49.784) (end 128.778 53.045196) (width 0.25) (layer "B.Cu") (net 4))
 (segment (start 128.778 69.977) (end 117.669196 69.977) (width 0.25) (layer "B.Cu") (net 4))
 (segment (start 128.778 53.045196) (end 128.778 69.977) (width 0.25) (layer "B.Cu") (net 4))
 (segment (start 117.669196 66.421) (end 137.481196 66.421) (width 0.25) (layer "F.Cu") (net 3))
 (segment (start 157.679196 86.619) (end 161.865196 86.619) (width 0.25) (layer "F.Cu") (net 3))
 (segment (start 137.481196 66.421) (end 157.679196 86.619) (width 0.25) (layer "F.Cu") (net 3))
 (segment (start 127.039196 66.333196) (end 127.127 66.421) (width 0.25) (layer "B.Cu") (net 3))
 (segment (start 127.039196 49.784) (end 127.039196 66.333196) (width 0.25) (layer "B.Cu") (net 3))
 (segment (start 127.127 66.421) (end 117.669196 66.421) (width 0.25) (layer "B.Cu") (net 3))
 (segment (start 117.669196 59.309) (end 140.095196 59.309) (width 0.25) (layer "F.Cu") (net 1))
 (segment (start 117.039196 49.784) (end 117.039196 58.679) (width 0.25) (layer "F.Cu") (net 1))
 (segment (start 140.095196 59.309) (end 161.865196 81.079) (width 0.25) (layer "F.Cu") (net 1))
 (segment (start 117.039196 58.679) (end 117.669196 59.309) (width 0.25) (layer "F.Cu") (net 1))
 (segment (start 158.846196 83.849) (end 161.865196 83.849) (width 0.25) (layer "F.Cu") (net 2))
 (segment (start 117.669196 62.865) (end 137.862196 62.865) (width 0.25) (layer "F.Cu") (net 2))
 (segment (start 137.862196 62.865) (end 158.846196 83.849) (width 0.25) (layer "F.Cu") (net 2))
 (segment (start 124.333 62.865) (end 117.669196 62.865) (width 0.25) (layer "B.Cu") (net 2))
 (segment (start 122.039196 49.784) (end 124.333 52.077804) (width 0.25) (layer "B.Cu") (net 2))
 (segment (start 124.333 52.077804) (end 124.333 62.865) (width 0.25) (layer "B.Cu") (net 2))
 (segment (start 156.958 152.781) (end 156.958 148.449) (width 0.25) (layer "F.Cu") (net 11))
 (segment (start 143.323196 94.869) (end 157.233196 108.779) (width 0.25) (layer "F.Cu") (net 11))
 (segment (start 123.825 115.062) (end 117.669196 115.062) (width 0.25) (layer "F.Cu") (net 11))
 (segment (start 124.333 115.57) (end 123.825 115.062) (width 0.25) (layer "F.Cu") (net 11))
 (segment (start 156.958 148.449) (end 124.333 115.824) (width 0.25) (layer "F.Cu") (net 11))
 (segment (start 117.669196 94.869) (end 143.323196 94.869) (width 0.25) (layer "F.Cu") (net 11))
 (segment (start 124.333 115.824) (end 124.333 115.57) (width 0.25) (layer "F.Cu") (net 11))
 (segment (start 157.233196 108.779) (end 161.865196 108.779) (width 0.25) (layer "F.Cu") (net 11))
 (segment (start 157.487 88.004) (end 164.405196 88.004) (width 0.25) (layer "B.Cu") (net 11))
 (segment (start 130.429 115.062) (end 157.487 88.004) (width 0.25) (layer "B.Cu") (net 11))
 (segment (start 167.039196 49.784) (end 135.89 80.933196) (width 0.25) (layer "B.Cu") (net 11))
 (segment (start 135.89 94.869) (end 117.669196 94.869) (width 0.25) (layer "B.Cu") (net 11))
 (segment (start 117.669196 115.062) (end 130.429 115.062) (width 0.25) (layer "B.Cu") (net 11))
 (segment (start 135.89 80.933196) (end 135.89 94.869) (width 0.25) (layer "B.Cu") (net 11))
 (segment (start 158.328196 114.319) (end 161.865196 114.319) (width 0.25) (layer "F.Cu") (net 13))
 (segment (start 120.126953 104.394) (end 121.904953 106.172) (width 0.25) (layer "F.Cu") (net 13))
 (segment (start 134.747 106.172) (end 171.958 143.383) (width 0.25) (layer "F.Cu") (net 13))
 (segment (start 121.904953 106.172) (end 134.747 106.172) (width 0.25) (layer "F.Cu") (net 13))
 (segment (start 171.958 143.383) (end 171.958 152.781) (width 0.25) (layer "F.Cu") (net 13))
 (segment (start 148.403196 104.394) (end 158.328196 114.319) (width 0.25) (layer "F.Cu") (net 13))
 (segment (start 117.669196 104.394) (end 148.403196 104.394) (width 0.25) (layer "F.Cu") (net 13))
 (segment (start 117.669196 104.394) (end 120.126953 104.394) (width 0.25) (layer "F.Cu") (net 13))
 (segment (start 166.958 143.43) (end 166.958 152.781) (width 0.25) (layer "F.Cu") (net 14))
 (segment (start 167.005 143.383) (end 166.958 143.43) (width 0.25) (layer "F.Cu") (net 14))
 (segment (start 117.669196 107.95) (end 131.572 107.95) (width 0.25) (layer "F.Cu") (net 14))
 (segment (start 131.572 107.95) (end 167.005 143.383) (width 0.25) (layer "F.Cu") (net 14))
 (segment (start 158.918 82.464) (end 164.405196 82.464) (width 0.25) (layer "B.Cu") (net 14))
 (segment (start 158.877 82.423) (end 158.918 82.464) (width 0.25) (layer "B.Cu") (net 14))
 (segment (start 117.669196 107.95) (end 133.35 107.95) (width 0.25) (layer "B.Cu") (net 14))
 (segment (start 133.35 107.95) (end 158.877 82.423) (width 0.25) (layer "B.Cu") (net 14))
 (segment (start 161.958 145.382) (end 161.958 152.781) (width 0.25) (layer "F.Cu") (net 15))
 (segment (start 128.27 111.506) (end 162.052 145.288) (width 0.25) (layer "F.Cu") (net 15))
 (segment (start 117.669196 111.506) (end 128.27 111.506) (width 0.25) (layer "F.Cu") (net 15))
 (segment (start 162.052 145.288) (end 161.958 145.382) (width 0.25) (layer "F.Cu") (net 15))
 (segment (start 158.369 85.217) (end 158.386 85.234) (width 0.25) (layer "B.Cu") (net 15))
 (segment (start 132.08 111.506) (end 158.369 85.217) (width 0.25) (layer "B.Cu") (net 15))
 (segment (start 158.386 85.234) (end 164.405196 85.234) (width 0.25) (layer "B.Cu") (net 15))
 (segment (start 117.669196 111.506) (end 132.08 111.506) (width 0.25) (layer "B.Cu") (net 15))
 (segment (start 123.063 118.618) (end 117.669196 118.618) (width 0.25) (layer "F.Cu") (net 16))
 (segment (start 151.958 147.513) (end 123.063 118.618) (width 0.25) (layer "F.Cu") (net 16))
 (segment (start 151.958 152.781) (end 151.958 147.513) (width 0.25) (layer "F.Cu") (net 16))
 (segment (start 117.669196 118.618) (end 129.667 118.618) (width 0.25) (layer "B.Cu") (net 16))
 (segment (start 157.703 90.774) (end 164.405196 90.774) (width 0.25) (layer "B.Cu") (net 16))
 (segment (start 157.607 90.678) (end 157.703 90.774) (width 0.25) (layer "B.Cu") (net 16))
 (segment (start 129.667 118.618) (end 157.607 90.678) (width 0.25) (layer "B.Cu") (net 16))
 (segment (start 121.666 122.174) (end 146.958 147.466) (width 0.25) (layer "F.Cu") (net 17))
 (segment (start 146.958 147.466) (end 146.958 152.781) (width 0.25) (layer "F.Cu") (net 17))
 (segment (start 117.669196 122.174) (end 121.666 122.174) (width 0.25) (layer "F.Cu") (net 17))
 (segment (start 117.669196 122.174) (end 127.889 122.174) (width 0.25) (layer "B.Cu") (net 17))
 (segment (start 127.889 122.174) (end 156.519 93.544) (width 0.25) (layer "B.Cu") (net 17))
 (segment (start 156.519 93.544) (end 164.405196 93.544) (width 0.25) (layer "B.Cu") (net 17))
 (segment (start 140.716 144.145) (end 141.097 144.145) (width 0.25) (layer "F.Cu") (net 18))
 (segment (start 122.301 125.73) (end 140.716 144.145) (width 0.25) (layer "F.Cu") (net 18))
 (segment (start 141.958 145.006) (end 141.958 152.781) (width 0.25) (layer "F.Cu") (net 18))
 (segment (start 117.669196 125.73) (end 122.301 125.73) (width 0.25) (layer "F.Cu") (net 18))
 (segment (start 141.097 144.145) (end 141.958 145.006) (width 0.25) (layer "F.Cu") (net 18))
 (segment (start 126.873 125.73) (end 156.289 96.314) (width 0.25) (layer "B.Cu") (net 18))
 (segment (start 156.289 96.314) (end 164.405196 96.314) (width 0.25) (layer "B.Cu") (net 18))
 (segment (start 117.669196 125.73) (end 126.873 125.73) (width 0.25) (layer "B.Cu") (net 18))
 (segment (start 123.317 129.286) (end 117.669196 129.286) (width 0.25) (layer "F.Cu") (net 19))
 (segment (start 136.958 142.927) (end 123.317 129.286) (width 0.25) (layer "F.Cu") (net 19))
 (segment (start 136.958 152.781) (end 136.958 142.927) (width 0.25) (layer "F.Cu") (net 19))
 (segment (start 125.857 129.286) (end 156.083 99.06) (width 0.25) (layer "B.Cu") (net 19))
 (segment (start 156.107 99.084) (end 164.405196 99.084) (width 0.25) (layer "B.Cu") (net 19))
 (segment (start 156.083 99.06) (end 156.107 99.084) (width 0.25) (layer "B.Cu") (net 19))
 (segment (start 117.669196 129.286) (end 125.857 129.286) (width 0.25) (layer "B.Cu") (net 19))
 (segment (start 123.571 132.842) (end 117.669196 132.842) (width 0.25) (layer "F.Cu") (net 20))
 (segment (start 131.958 141.229) (end 123.571 132.842) (width 0.25) (layer "F.Cu") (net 20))
 (segment (start 131.958 152.781) (end 131.958 141.229) (width 0.25) (layer "F.Cu") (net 20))
 (segment (start 125.095 132.842) (end 156.083 101.854) (width 0.25) (layer "B.Cu") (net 20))
 (segment (start 156.083 101.854) (end 164.405196 101.854) (width 0.25) (layer "B.Cu") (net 20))
 (segment (start 117.669196 132.842) (end 125.095 132.842) (width 0.25) (layer "B.Cu") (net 20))
 (segment (start 126.958 140.674) (end 122.682 136.398) (width 0.25) (layer "F.Cu") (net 21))
 (segment (start 122.682 136.398) (end 117.669196 136.398) (width 0.25) (layer "F.Cu") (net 21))
 (segment (start 126.958 152.781) (end 126.958 140.674) (width 0.25) (layer "F.Cu") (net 21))
 (segment (start 117.669196 136.398) (end 124.841 136.398) (width 0.25) (layer "B.Cu") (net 21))
 (segment (start 124.841 136.398) (end 156.615 104.624) (width 0.25) (layer "B.Cu") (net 21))
 (segment (start 156.615 104.624) (end 164.405196 104.624) (width 0.25) (layer "B.Cu") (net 21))
 (segment (start 116.958 152.781) (end 116.958 144.221196) (width 0.25) (layer "F.Cu") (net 23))
 (segment (start 116.958 144.221196) (end 117.669196 143.51) (width 0.25) (layer "F.Cu") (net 23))
 (segment (start 158.695 110.164) (end 164.405196 110.164) (width 0.25) (layer "B.Cu") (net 23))
 (segment (start 117.669196 143.51) (end 125.349 143.51) (width 0.25) (layer "B.Cu") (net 23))
 (segment (start 125.349 143.51) (end 158.695 110.164) (width 0.25) (layer "B.Cu") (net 23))
 (segment (start 121.958 152.781) (end 124.968 149.771) (width 0.25) (layer "F.Cu") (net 22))
 (segment (start 124.968 141.605) (end 123.317 139.954) (width 0.25) (layer "F.Cu") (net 22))
 (segment (start 123.317 139.954) (end 117.669196 139.954) (width 0.25) (layer "F.Cu") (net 22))
 (segment (start 124.968 149.771) (end 124.968 141.605) (width 0.25) (layer "F.Cu") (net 22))
 (segment (start 156.766 107.394) (end 164.405196 107.394) (width 0.25) (layer "B.Cu") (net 22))
 (segment (start 117.669196 139.954) (end 124.206 139.954) (width 0.25) (layer "B.Cu") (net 22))
 (segment (start 124.206 139.954) (end 156.766 107.394) (width 0.25) (layer "B.Cu") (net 22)))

